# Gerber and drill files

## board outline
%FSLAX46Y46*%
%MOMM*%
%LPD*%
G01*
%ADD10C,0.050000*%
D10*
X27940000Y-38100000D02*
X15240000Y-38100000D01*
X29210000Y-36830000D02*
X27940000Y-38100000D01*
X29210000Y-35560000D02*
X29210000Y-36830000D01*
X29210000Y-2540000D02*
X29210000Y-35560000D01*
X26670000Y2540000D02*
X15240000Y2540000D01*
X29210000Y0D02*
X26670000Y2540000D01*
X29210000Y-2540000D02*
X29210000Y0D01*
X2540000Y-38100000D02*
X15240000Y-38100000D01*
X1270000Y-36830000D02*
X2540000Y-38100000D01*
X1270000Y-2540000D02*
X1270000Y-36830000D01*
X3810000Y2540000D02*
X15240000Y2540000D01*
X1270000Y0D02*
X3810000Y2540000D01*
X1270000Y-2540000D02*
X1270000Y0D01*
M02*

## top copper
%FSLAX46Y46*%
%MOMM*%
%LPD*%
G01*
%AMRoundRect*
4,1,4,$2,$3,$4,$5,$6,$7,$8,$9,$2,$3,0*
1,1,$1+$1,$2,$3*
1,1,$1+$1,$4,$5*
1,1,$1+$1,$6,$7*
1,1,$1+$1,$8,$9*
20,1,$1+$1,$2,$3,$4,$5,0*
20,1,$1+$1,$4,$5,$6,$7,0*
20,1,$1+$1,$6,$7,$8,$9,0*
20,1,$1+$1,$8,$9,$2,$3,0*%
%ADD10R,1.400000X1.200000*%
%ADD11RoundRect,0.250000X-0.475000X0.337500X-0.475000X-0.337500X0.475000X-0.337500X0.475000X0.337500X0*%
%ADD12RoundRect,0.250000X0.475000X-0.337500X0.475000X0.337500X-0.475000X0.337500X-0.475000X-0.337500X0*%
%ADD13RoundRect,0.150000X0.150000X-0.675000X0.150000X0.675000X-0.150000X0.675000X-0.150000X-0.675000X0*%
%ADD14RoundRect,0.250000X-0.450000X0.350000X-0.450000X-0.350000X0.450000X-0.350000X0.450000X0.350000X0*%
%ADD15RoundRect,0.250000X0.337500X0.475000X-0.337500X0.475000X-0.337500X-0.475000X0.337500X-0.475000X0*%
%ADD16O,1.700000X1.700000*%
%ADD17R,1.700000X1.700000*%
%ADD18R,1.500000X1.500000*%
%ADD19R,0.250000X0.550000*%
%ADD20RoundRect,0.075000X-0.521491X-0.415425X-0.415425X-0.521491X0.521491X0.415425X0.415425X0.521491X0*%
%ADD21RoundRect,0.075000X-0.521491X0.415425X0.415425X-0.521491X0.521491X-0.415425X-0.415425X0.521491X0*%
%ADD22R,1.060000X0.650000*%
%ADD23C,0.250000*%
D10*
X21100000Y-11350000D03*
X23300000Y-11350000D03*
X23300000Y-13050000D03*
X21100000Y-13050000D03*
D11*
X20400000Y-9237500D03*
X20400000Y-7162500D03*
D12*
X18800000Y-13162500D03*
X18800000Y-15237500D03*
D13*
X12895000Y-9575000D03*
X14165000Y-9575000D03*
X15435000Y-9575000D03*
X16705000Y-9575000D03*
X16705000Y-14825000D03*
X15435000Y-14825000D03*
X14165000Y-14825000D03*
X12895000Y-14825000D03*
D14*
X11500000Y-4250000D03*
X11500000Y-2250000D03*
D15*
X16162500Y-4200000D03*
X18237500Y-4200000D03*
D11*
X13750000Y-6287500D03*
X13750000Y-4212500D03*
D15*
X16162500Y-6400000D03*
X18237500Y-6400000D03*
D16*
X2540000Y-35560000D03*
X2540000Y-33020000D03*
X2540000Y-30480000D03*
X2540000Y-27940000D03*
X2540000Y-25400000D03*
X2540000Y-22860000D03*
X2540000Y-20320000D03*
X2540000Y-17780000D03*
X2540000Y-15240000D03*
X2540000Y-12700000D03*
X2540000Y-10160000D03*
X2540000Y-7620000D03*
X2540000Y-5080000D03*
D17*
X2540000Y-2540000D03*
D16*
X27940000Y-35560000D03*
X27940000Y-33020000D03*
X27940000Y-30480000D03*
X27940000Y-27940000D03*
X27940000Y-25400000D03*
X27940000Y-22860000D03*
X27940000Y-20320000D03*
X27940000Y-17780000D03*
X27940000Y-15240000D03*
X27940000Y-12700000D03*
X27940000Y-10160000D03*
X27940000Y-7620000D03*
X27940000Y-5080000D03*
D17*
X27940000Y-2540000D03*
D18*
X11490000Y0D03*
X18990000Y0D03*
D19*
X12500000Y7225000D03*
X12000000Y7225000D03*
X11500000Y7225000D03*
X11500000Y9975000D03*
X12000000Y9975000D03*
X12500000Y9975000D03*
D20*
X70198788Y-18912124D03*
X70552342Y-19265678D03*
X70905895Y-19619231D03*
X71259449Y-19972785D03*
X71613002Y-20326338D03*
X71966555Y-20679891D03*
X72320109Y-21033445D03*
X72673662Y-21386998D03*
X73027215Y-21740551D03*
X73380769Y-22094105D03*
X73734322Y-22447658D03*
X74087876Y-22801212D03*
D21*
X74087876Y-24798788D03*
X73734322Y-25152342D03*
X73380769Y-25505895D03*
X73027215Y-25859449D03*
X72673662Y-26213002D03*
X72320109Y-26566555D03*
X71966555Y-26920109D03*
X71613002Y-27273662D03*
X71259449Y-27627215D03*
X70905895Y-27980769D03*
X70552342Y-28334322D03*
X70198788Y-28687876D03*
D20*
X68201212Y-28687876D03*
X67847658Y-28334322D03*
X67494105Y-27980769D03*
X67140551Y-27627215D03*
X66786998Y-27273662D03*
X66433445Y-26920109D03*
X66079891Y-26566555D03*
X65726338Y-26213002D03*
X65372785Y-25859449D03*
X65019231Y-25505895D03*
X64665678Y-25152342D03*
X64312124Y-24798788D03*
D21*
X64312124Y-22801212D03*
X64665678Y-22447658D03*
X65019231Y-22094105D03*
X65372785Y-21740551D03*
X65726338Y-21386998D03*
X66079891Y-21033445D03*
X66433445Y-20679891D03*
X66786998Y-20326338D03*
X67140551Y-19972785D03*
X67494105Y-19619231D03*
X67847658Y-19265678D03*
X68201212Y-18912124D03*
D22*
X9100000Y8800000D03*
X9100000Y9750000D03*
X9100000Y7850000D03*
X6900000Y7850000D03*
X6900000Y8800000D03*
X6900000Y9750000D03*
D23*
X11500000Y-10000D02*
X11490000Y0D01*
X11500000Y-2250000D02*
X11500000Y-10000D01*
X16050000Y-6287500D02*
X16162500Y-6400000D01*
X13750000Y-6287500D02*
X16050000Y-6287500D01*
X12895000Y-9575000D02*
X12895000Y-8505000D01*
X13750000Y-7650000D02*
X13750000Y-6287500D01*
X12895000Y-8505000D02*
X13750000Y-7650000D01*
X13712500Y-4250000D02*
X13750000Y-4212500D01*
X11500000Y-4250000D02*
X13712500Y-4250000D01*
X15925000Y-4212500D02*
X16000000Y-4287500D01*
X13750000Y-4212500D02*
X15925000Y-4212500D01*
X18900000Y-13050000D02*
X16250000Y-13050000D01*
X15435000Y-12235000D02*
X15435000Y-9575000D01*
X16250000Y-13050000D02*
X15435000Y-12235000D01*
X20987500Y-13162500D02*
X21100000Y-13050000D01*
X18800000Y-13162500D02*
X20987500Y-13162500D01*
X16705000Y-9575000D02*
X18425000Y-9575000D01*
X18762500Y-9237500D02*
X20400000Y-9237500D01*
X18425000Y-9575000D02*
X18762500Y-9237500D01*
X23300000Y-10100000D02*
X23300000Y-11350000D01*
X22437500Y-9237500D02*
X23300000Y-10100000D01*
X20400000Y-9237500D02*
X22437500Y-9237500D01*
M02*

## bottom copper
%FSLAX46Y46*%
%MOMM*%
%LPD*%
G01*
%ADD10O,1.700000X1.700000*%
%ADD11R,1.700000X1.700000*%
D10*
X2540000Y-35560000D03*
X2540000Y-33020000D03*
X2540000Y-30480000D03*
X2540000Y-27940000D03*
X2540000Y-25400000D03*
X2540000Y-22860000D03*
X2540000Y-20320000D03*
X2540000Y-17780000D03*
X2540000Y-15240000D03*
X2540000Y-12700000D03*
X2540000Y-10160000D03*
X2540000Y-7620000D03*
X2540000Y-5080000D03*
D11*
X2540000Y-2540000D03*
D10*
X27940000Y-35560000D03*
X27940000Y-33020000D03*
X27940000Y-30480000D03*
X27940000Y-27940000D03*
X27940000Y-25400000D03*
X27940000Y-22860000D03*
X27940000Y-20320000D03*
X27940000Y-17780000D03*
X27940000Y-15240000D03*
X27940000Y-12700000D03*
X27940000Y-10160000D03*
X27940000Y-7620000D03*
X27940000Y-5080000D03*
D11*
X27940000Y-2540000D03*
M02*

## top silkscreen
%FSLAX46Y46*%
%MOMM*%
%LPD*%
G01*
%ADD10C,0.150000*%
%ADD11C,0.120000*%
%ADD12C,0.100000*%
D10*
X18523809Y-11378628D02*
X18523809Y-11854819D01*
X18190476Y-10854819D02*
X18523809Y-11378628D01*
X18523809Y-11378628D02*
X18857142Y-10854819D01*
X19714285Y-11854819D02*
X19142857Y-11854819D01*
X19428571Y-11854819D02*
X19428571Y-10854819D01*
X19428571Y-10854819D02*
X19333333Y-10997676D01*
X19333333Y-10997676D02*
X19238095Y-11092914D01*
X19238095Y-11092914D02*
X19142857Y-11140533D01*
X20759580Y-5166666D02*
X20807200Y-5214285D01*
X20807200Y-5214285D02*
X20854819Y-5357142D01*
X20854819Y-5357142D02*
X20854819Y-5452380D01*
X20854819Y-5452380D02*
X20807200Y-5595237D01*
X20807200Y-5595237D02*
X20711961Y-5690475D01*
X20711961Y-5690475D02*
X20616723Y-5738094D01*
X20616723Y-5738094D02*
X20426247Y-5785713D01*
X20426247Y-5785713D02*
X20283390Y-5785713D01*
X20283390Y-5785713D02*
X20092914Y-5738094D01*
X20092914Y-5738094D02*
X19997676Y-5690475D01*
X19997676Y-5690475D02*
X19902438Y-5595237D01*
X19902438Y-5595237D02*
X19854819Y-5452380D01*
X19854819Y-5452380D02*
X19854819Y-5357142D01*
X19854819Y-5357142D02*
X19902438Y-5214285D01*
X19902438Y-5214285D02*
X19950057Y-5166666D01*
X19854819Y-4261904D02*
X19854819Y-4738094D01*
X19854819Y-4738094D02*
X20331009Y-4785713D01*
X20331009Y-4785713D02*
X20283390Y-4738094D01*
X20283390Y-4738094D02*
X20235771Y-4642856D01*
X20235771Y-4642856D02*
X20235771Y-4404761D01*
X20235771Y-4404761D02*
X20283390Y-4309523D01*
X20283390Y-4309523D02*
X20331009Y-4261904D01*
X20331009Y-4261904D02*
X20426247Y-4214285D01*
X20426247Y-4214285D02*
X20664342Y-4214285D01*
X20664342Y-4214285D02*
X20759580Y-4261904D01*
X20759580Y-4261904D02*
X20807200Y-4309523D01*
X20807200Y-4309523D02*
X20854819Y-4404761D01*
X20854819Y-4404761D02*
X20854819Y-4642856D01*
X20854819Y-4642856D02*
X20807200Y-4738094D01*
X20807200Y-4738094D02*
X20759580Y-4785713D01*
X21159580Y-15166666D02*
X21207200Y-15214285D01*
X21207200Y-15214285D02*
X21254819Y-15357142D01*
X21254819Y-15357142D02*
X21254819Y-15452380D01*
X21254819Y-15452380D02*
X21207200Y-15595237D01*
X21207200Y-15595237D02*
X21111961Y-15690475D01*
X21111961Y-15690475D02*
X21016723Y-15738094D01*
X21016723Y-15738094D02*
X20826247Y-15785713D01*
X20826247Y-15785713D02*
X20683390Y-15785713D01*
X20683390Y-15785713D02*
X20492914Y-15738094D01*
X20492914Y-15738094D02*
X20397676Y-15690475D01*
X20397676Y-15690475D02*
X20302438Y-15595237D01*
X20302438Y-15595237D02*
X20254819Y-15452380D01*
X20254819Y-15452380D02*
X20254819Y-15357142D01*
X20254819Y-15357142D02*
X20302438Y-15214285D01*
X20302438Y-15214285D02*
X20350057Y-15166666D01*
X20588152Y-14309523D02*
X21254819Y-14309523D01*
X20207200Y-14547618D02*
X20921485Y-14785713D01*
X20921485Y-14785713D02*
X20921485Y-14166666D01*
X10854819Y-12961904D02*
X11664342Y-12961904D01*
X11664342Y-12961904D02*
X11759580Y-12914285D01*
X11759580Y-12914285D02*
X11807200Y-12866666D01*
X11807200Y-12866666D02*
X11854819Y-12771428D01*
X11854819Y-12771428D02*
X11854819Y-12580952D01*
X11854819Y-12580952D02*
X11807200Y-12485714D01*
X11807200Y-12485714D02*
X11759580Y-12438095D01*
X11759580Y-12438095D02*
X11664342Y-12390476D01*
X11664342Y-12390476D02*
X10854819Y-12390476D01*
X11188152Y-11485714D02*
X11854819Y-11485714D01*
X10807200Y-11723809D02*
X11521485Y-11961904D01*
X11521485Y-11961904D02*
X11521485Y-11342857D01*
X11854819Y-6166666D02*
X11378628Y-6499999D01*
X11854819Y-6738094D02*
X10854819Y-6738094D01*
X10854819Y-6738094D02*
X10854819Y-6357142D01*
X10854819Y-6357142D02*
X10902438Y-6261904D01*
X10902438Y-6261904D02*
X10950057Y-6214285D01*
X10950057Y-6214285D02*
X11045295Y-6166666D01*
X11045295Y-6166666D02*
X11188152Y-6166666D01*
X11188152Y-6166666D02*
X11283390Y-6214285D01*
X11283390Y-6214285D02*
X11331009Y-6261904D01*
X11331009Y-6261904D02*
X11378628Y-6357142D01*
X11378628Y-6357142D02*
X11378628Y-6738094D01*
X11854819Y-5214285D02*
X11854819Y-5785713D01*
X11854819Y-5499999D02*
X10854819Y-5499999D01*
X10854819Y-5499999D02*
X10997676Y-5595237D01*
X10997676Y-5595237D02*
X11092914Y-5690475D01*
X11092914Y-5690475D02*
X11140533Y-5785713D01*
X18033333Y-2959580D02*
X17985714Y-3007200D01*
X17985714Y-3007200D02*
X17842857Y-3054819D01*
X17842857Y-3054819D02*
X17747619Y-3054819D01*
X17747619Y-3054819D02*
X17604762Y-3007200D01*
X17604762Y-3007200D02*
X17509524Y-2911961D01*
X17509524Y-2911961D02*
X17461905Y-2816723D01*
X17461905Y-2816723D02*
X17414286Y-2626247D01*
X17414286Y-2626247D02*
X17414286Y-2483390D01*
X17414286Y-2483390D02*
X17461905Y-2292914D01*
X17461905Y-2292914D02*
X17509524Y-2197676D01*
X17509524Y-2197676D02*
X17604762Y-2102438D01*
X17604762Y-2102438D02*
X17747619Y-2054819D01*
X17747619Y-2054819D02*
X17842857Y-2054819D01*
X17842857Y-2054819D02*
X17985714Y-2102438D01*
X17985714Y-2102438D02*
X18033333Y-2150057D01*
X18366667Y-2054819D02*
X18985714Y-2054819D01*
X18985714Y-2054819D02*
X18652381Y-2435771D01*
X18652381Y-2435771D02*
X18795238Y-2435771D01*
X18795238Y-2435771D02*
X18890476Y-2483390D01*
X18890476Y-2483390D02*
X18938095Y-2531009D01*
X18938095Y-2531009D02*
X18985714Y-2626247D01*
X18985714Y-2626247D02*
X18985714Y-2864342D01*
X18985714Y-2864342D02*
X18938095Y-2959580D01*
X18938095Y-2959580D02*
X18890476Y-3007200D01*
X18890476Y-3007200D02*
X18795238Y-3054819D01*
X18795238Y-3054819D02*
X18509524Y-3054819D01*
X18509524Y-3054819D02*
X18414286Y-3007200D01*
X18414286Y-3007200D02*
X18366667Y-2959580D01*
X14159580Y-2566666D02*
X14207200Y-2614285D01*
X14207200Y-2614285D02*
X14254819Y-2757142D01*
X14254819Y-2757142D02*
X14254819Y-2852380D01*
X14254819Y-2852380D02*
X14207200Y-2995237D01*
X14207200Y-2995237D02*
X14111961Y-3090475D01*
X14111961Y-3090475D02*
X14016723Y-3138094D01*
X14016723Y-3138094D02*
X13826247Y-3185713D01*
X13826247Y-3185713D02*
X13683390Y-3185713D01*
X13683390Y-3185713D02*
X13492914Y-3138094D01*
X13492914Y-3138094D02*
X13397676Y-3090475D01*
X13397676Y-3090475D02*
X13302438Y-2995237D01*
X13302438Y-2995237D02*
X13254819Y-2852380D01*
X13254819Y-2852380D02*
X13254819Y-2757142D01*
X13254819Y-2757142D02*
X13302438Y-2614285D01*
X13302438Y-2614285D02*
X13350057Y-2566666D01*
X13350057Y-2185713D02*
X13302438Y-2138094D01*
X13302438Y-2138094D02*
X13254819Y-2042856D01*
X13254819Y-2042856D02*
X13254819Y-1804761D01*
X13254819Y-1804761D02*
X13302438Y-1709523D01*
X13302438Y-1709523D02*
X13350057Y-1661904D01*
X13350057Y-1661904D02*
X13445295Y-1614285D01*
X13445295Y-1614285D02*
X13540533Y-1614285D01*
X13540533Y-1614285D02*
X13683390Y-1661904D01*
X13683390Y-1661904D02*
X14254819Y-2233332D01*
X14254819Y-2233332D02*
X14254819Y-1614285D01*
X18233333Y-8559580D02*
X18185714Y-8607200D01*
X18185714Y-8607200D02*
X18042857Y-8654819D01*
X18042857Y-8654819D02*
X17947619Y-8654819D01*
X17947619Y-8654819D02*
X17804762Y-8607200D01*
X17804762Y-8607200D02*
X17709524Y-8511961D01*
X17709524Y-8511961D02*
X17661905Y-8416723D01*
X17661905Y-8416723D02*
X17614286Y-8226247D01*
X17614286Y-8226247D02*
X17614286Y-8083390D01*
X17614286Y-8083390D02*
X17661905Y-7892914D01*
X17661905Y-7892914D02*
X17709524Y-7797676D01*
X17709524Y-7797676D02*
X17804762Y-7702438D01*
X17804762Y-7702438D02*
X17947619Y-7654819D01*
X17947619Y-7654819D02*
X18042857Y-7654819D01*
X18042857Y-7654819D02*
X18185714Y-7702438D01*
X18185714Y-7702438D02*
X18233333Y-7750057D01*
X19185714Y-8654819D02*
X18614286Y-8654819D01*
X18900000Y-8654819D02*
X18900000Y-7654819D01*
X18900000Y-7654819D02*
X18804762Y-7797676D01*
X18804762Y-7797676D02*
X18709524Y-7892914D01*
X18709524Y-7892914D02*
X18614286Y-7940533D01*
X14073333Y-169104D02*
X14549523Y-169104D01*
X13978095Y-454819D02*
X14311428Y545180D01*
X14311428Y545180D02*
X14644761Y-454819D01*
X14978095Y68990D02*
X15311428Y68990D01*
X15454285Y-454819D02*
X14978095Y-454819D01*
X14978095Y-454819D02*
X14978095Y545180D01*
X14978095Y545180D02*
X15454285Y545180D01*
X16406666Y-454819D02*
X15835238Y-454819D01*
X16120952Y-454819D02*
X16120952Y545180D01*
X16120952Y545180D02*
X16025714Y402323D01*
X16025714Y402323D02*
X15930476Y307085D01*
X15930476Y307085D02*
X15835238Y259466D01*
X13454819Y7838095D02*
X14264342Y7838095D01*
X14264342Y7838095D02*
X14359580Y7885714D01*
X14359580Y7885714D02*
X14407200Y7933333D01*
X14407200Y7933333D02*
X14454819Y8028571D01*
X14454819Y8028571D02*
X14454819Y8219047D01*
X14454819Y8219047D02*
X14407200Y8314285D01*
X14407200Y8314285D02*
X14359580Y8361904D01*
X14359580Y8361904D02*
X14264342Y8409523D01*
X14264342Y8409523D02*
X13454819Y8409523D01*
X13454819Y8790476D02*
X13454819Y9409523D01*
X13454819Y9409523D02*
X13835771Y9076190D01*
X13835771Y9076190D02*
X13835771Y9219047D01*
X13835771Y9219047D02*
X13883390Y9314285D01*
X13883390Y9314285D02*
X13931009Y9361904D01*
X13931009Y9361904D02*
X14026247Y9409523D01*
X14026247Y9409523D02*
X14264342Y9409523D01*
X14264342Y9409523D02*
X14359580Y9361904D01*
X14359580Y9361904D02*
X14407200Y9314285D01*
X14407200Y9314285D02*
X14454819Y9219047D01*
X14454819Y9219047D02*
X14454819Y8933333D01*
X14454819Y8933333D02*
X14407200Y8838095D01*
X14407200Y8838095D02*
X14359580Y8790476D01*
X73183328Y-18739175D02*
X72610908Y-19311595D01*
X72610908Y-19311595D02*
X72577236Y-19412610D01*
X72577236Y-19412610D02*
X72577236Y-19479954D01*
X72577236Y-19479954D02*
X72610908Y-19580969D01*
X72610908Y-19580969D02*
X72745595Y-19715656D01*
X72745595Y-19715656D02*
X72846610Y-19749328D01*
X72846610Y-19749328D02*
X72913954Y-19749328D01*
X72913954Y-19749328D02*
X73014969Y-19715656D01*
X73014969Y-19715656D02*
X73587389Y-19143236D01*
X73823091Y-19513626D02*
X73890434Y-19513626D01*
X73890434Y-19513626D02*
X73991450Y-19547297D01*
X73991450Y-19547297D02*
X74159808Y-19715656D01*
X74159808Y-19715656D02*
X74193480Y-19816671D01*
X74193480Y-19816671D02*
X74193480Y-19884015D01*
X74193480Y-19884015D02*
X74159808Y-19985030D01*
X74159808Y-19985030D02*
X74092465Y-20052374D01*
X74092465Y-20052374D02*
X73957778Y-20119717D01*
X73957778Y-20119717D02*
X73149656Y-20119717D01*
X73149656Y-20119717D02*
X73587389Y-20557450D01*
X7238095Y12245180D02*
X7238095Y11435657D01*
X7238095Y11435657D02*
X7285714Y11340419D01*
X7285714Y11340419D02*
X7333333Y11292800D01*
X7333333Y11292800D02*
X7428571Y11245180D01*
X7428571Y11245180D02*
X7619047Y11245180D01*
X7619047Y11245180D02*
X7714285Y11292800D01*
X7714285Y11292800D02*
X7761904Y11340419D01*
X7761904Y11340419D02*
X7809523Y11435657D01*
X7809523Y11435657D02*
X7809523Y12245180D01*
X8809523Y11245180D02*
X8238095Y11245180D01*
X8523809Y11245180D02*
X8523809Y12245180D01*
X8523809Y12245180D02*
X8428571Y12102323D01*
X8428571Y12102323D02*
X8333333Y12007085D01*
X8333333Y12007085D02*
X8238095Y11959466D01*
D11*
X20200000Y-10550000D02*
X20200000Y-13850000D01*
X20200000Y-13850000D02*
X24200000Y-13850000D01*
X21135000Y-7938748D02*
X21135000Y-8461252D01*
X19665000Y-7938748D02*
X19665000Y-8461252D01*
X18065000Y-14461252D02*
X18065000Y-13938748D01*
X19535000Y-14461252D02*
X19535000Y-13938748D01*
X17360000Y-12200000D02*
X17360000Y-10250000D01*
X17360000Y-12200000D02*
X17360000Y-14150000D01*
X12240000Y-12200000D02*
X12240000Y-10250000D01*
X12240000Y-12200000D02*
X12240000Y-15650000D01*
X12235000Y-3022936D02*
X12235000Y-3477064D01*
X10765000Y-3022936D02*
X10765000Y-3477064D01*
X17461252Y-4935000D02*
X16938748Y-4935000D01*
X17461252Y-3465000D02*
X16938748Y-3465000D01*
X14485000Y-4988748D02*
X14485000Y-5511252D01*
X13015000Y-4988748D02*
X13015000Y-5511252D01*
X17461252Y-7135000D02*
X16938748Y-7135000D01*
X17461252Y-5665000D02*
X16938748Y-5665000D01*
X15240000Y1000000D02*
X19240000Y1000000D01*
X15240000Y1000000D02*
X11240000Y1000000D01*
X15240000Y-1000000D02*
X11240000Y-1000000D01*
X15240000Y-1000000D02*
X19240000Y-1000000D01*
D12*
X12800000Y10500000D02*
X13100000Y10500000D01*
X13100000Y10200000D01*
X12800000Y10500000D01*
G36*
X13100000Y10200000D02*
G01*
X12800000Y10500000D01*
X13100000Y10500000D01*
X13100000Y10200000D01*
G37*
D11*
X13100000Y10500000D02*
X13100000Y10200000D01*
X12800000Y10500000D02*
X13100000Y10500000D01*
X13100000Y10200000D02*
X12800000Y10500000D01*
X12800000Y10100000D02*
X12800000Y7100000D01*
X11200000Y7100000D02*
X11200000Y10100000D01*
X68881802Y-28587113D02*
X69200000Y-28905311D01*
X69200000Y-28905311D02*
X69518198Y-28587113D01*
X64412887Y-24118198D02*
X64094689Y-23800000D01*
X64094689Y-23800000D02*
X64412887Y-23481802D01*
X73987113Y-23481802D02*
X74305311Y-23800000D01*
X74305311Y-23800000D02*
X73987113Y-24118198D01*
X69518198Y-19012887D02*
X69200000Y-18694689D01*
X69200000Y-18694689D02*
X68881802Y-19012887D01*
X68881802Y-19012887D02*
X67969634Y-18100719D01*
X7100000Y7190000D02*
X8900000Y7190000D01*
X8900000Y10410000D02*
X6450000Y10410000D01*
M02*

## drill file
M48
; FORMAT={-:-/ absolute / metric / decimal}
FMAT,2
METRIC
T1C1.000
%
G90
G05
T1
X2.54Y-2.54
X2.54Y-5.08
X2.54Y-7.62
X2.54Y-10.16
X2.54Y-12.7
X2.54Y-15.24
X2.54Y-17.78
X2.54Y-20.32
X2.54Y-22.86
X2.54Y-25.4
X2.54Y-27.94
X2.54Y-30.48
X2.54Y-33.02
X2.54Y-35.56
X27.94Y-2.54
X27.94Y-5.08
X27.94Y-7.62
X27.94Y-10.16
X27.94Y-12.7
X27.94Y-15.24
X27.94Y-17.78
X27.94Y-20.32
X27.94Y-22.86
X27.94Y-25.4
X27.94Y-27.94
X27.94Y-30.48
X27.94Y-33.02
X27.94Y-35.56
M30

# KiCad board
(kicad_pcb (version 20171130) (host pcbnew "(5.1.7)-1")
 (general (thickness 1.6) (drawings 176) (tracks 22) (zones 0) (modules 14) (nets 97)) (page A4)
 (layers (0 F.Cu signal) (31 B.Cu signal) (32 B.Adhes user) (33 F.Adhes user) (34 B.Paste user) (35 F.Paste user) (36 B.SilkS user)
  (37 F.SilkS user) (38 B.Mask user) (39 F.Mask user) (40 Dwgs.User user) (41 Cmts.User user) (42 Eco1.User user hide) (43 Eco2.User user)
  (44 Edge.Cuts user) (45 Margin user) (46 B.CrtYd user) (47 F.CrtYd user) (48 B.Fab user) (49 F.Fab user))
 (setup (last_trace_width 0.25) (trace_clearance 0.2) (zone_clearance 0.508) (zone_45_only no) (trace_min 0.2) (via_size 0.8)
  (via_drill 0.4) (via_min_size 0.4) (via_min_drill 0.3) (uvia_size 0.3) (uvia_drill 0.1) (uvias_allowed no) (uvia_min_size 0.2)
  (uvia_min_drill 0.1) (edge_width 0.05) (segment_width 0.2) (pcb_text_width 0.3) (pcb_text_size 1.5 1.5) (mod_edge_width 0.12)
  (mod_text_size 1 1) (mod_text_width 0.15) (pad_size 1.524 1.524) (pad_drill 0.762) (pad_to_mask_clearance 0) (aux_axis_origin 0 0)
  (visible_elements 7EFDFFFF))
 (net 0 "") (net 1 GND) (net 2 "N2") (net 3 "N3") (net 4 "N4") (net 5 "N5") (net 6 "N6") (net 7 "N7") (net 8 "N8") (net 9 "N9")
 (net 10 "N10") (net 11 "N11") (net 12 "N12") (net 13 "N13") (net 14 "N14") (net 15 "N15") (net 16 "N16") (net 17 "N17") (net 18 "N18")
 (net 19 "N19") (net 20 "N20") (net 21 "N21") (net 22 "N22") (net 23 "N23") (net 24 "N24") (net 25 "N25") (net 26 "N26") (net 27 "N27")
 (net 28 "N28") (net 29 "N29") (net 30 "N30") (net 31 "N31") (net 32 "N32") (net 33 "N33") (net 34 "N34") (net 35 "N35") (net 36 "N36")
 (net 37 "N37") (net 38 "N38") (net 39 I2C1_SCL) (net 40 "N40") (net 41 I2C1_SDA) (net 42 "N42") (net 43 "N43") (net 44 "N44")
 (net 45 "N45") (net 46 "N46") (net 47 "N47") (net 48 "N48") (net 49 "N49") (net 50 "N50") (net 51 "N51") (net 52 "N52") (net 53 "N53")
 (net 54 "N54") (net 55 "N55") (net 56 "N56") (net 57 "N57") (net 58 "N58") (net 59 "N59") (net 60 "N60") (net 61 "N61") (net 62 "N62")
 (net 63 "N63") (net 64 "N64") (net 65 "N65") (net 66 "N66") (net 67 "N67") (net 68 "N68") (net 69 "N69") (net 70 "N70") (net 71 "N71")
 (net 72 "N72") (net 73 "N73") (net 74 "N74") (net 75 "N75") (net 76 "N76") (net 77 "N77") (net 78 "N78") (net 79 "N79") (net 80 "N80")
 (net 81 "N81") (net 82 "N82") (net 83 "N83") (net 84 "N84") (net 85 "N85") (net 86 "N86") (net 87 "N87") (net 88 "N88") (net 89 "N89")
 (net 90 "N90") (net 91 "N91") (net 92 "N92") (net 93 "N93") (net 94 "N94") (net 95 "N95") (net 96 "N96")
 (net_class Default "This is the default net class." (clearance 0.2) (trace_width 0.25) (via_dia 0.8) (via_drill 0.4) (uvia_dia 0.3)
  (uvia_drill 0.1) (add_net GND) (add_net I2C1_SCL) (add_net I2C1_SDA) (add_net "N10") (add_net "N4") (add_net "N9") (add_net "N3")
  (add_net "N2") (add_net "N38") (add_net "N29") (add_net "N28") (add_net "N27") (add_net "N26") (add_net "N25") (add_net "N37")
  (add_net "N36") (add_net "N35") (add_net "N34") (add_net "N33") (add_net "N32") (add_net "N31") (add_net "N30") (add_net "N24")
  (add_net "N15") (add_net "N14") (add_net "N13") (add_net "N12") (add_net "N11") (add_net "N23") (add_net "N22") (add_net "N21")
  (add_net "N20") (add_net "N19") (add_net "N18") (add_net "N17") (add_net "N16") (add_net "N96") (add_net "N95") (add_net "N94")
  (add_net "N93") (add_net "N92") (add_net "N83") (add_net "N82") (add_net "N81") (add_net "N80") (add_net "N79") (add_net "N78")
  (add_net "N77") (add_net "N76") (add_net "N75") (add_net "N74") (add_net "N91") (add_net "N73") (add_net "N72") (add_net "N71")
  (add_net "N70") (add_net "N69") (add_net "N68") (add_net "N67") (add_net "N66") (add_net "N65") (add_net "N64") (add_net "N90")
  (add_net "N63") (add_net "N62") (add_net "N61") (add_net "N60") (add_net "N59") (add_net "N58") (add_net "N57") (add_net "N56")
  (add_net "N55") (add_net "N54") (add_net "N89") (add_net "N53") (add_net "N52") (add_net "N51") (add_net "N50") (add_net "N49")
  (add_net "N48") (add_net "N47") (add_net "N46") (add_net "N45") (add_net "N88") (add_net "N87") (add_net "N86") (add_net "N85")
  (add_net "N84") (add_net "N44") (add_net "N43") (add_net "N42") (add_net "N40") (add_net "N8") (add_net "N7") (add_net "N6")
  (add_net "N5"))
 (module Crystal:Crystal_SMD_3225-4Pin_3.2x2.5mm (layer F.Cu) (at 22.2 12.2)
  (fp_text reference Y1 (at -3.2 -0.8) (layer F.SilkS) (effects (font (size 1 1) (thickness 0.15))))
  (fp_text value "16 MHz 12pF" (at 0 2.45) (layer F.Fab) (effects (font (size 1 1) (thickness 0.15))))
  (fp_line (start -2 -1.65) (end -2 1.65) (layer F.SilkS) (width 0.12))
  (fp_line (start -2 1.65) (end 2 1.65) (layer F.SilkS) (width 0.12))
  (pad 4 smd rect (at -1.1 -0.85) (size 1.4 1.2) (layers F.Cu F.Paste F.Mask) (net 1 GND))
  (pad 3 smd rect (at 1.1 -0.85) (size 1.4 1.2) (layers F.Cu F.Paste F.Mask) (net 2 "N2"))
  (pad 2 smd rect (at 1.1 0.85) (size 1.4 1.2) (layers F.Cu F.Paste F.Mask) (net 1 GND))
  (pad 1 smd rect (at -1.1 0.85) (size 1.4 1.2) (layers F.Cu F.Paste F.Mask) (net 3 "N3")))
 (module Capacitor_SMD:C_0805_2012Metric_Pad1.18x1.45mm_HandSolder (layer F.Cu) (at 20.4 8.2 270)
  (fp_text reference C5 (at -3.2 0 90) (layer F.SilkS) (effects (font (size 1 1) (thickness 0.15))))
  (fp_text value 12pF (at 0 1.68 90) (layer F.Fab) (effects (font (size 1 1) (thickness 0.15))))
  (fp_line (start -0.261252 -0.735) (end 0.261252 -0.735) (layer F.SilkS) (width 0.12))
  (fp_line (start -0.261252 0.735) (end 0.261252 0.735) (layer F.SilkS) (width 0.12))
  (pad 2 smd roundrect (at 1.0375 0 270) (size 1.175 1.45) (layers F.Cu F.Paste F.Mask) (roundrect_rratio 0.212766) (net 2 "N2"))
  (pad 1 smd roundrect (at -1.0375 0 270) (size 1.175 1.45) (layers F.Cu F.Paste F.Mask) (roundrect_rratio 0.212766) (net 1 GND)))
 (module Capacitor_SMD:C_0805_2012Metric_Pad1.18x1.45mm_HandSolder (layer F.Cu) (at 18.8 14.2 90)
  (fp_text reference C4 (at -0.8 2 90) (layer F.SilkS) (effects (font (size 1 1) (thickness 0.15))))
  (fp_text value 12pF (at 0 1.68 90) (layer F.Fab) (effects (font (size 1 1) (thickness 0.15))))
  (fp_line (start -0.261252 -0.735) (end 0.261252 -0.735) (layer F.SilkS) (width 0.12))
  (fp_line (start -0.261252 0.735) (end 0.261252 0.735) (layer F.SilkS) (width 0.12))
  (pad 2 smd roundrect (at 1.0375 0 90) (size 1.175 1.45) (layers F.Cu F.Paste F.Mask) (roundrect_rratio 0.212766) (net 3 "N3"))
  (pad 1 smd roundrect (at -1.0375 0 90) (size 1.175 1.45) (layers F.Cu F.Paste F.Mask) (roundrect_rratio 0.212766) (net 1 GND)))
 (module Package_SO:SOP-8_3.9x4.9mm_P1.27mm (layer F.Cu) (at 14.8 12.2 90)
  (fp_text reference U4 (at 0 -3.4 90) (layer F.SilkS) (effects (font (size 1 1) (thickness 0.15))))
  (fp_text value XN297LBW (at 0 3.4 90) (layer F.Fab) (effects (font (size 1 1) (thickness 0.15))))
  (fp_line (start 0 2.56) (end 1.95 2.56) (layer F.SilkS) (width 0.12))
  (fp_line (start 0 2.56) (end -1.95 2.56) (layer F.SilkS) (width 0.12))
  (fp_line (start 0 -2.56) (end 1.95 -2.56) (layer F.SilkS) (width 0.12))
  (fp_line (start 0 -2.56) (end -3.45 -2.56) (layer F.SilkS) (width 0.12))
  (pad 8 smd roundrect (at 2.625 -1.905 90) (size 1.65 0.6) (layers F.Cu F.Paste F.Mask) (roundrect_rratio 0.25) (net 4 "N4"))
  (pad 7 smd roundrect (at 2.625 -0.635 90) (size 1.65 0.6) (layers F.Cu F.Paste F.Mask) (roundrect_rratio 0.25) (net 1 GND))
  (pad 6 smd roundrect (at 2.625 0.635 90) (size 1.65 0.6) (layers F.Cu F.Paste F.Mask) (roundrect_rratio 0.25) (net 3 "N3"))
  (pad 5 smd roundrect (at 2.625 1.905 90) (size 1.65 0.6) (layers F.Cu F.Paste F.Mask) (roundrect_rratio 0.25) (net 2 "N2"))
  (pad 4 smd roundrect (at -2.625 1.905 90) (size 1.65 0.6) (layers F.Cu F.Paste F.Mask) (roundrect_rratio 0.25) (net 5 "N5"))
  (pad 3 smd roundrect (at -2.625 0.635 90) (size 1.65 0.6) (layers F.Cu F.Paste F.Mask) (roundrect_rratio 0.25) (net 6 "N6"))
  (pad 2 smd roundrect (at -2.625 -0.635 90) (size 1.65 0.6) (layers F.Cu F.Paste F.Mask) (roundrect_rratio 0.25) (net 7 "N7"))
  (pad 1 smd roundrect (at -2.625 -1.905 90) (size 1.65 0.6) (layers F.Cu F.Paste F.Mask) (roundrect_rratio 0.25) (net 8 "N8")))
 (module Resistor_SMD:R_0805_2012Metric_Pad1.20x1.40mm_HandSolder (layer F.Cu) (at 11.5 3.25 270)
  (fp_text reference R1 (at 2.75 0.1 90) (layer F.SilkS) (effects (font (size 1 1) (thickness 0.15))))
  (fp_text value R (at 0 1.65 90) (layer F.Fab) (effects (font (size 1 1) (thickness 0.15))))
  (fp_line (start -0.227064 -0.735) (end 0.227064 -0.735) (layer F.SilkS) (width 0.12))
  (fp_line (start -0.227064 0.735) (end 0.227064 0.735) (layer F.SilkS) (width 0.12))
  (pad 2 smd roundrect (at 1 0 270) (size 1.2 1.4) (layers F.Cu F.Paste F.Mask) (roundrect_rratio 0.208333) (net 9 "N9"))
  (pad 1 smd roundrect (at -1 0 270) (size 1.2 1.4) (layers F.Cu F.Paste F.Mask) (roundrect_rratio 0.208333) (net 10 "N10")))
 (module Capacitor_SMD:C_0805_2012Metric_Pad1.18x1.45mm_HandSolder (layer F.Cu) (at 17.2 4.2 180)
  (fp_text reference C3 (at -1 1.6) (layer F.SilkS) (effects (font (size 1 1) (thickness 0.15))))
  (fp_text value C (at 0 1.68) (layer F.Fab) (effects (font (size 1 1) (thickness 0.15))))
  (fp_line (start -0.261252 -0.735) (end 0.261252 -0.735) (layer F.SilkS) (width 0.12))
  (fp_line (start -0.261252 0.735) (end 0.261252 0.735) (layer F.SilkS) (width 0.12))
  (pad 2 smd roundrect (at 1.0375 0 180) (size 1.175 1.45) (layers F.Cu F.Paste F.Mask) (roundrect_rratio 0.212766) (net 9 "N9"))
  (pad 1 smd roundrect (at -1.0375 0 180) (size 1.175 1.45) (layers F.Cu F.Paste F.Mask) (roundrect_rratio 0.212766) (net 1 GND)))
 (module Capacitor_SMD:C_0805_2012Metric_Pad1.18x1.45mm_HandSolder (layer F.Cu) (at 13.75 5.25 270)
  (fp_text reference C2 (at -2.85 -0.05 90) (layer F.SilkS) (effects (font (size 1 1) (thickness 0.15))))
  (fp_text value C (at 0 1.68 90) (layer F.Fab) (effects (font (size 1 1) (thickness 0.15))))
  (fp_line (start -0.261252 -0.735) (end 0.261252 -0.735) (layer F.SilkS) (width 0.12))
  (fp_line (start -0.261252 0.735) (end 0.261252 0.735) (layer F.SilkS) (width 0.12))
  (pad 2 smd roundrect (at 1.0375 0 270) (size 1.175 1.45) (layers F.Cu F.Paste F.Mask) (roundrect_rratio 0.212766) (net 4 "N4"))
  (pad 1 smd roundrect (at -1.0375 0 270) (size 1.175 1.45) (layers F.Cu F.Paste F.Mask) (roundrect_rratio 0.212766) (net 9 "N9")))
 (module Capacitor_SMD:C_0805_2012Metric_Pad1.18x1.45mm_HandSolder (layer F.Cu) (at 17.2 6.4 180)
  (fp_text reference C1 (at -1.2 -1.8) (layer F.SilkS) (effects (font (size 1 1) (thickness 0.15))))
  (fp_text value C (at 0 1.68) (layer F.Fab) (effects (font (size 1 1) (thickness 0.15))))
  (fp_line (start -0.261252 -0.735) (end 0.261252 -0.735) (layer F.SilkS) (width 0.12))
  (fp_line (start -0.261252 0.735) (end 0.261252 0.735) (layer F.SilkS) (width 0.12))
  (pad 2 smd roundrect (at 1.0375 0 180) (size 1.175 1.45) (layers F.Cu F.Paste F.Mask) (roundrect_rratio 0.212766) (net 4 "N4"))
  (pad 1 smd roundrect (at -1.0375 0 180) (size 1.175 1.45) (layers F.Cu F.Paste F.Mask) (roundrect_rratio 0.212766) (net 1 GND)))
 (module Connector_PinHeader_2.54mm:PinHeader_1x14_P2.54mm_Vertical (layer B.Cu) (at 2.54 2.54 180)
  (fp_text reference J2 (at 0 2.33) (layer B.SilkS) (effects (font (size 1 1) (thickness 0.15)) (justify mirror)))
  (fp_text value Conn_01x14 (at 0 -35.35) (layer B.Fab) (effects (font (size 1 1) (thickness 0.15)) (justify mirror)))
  (pad 14 thru_hole oval (at 0 -33.02 180) (size 1.7 1.7) (drill 1) (layers *.Cu *.Mask) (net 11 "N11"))
  (pad 13 thru_hole oval (at 0 -30.48 180) (size 1.7 1.7) (drill 1) (layers *.Cu *.Mask) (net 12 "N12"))
  (pad 12 thru_hole oval (at 0 -27.94 180) (size 1.7 1.7) (drill 1) (layers *.Cu *.Mask) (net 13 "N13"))
  (pad 11 thru_hole oval (at 0 -25.4 180) (size 1.7 1.7) (drill 1) (layers *.Cu *.Mask) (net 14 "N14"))
  (pad 10 thru_hole oval (at 0 -22.86 180) (size 1.7 1.7) (drill 1) (layers *.Cu *.Mask) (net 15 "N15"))
  (pad 9 thru_hole oval (at 0 -20.32 180) (size 1.7 1.7) (drill 1) (layers *.Cu *.Mask) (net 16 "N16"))
  (pad 8 thru_hole oval (at 0 -17.78 180) (size 1.7 1.7) (drill 1) (layers *.Cu *.Mask) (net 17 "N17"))
  (pad 7 thru_hole oval (at 0 -15.24 180) (size 1.7 1.7) (drill 1) (layers *.Cu *.Mask) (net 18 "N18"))
  (pad 6 thru_hole oval (at 0 -12.7 180) (size 1.7 1.7) (drill 1) (layers *.Cu *.Mask) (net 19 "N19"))
  (pad 5 thru_hole oval (at 0 -10.16 180) (size 1.7 1.7) (drill 1) (layers *.Cu *.Mask) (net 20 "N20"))
  (pad 4 thru_hole oval (at 0 -7.62 180) (size 1.7 1.7) (drill 1) (layers *.Cu *.Mask) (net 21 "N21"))
  (pad 3 thru_hole oval (at 0 -5.08 180) (size 1.7 1.7) (drill 1) (layers *.Cu *.Mask) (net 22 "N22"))
  (pad 2 thru_hole oval (at 0 -2.54 180) (size 1.7 1.7) (drill 1) (layers *.Cu *.Mask) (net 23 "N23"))
  (pad 1 thru_hole rect (at 0 0 180) (size 1.7 1.7) (drill 1) (layers *.Cu *.Mask) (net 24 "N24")))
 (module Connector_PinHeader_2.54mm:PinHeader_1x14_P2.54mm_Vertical (layer B.Cu) (at 27.94 2.54 180)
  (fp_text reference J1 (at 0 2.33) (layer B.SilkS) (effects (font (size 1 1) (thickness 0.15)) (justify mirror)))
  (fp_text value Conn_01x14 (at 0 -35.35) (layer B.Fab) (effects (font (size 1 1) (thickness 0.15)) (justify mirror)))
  (pad 14 thru_hole oval (at 0 -33.02 180) (size 1.7 1.7) (drill 1) (layers *.Cu *.Mask) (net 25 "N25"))
  (pad 13 thru_hole oval (at 0 -30.48 180) (size 1.7 1.7) (drill 1) (layers *.Cu *.Mask) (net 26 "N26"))
  (pad 12 thru_hole oval (at 0 -27.94 180) (size 1.7 1.7) (drill 1) (layers *.Cu *.Mask) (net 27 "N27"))
  (pad 11 thru_hole oval (at 0 -25.4 180) (size 1.7 1.7) (drill 1) (layers *.Cu *.Mask) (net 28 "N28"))
  (pad 10 thru_hole oval (at 0 -22.86 180) (size 1.7 1.7) (drill 1) (layers *.Cu *.Mask) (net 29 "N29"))
  (pad 9 thru_hole oval (at 0 -20.32 180) (size 1.7 1.7) (drill 1) (layers *.Cu *.Mask) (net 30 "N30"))
  (pad 8 thru_hole oval (at 0 -17.78 180) (size 1.7 1.7) (drill 1) (layers *.Cu *.Mask) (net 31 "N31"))
  (pad 7 thru_hole oval (at 0 -15.24 180) (size 1.7 1.7) (drill 1) (layers *.Cu *.Mask) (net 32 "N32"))
  (pad 6 thru_hole oval (at 0 -12.7 180) (size 1.7 1.7) (drill 1) (layers *.Cu *.Mask) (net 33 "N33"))
  (pad 5 thru_hole oval (at 0 -10.16 180) (size 1.7 1.7) (drill 1) (layers *.Cu *.Mask) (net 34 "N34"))
  (pad 4 thru_hole oval (at 0 -7.62 180) (size 1.7 1.7) (drill 1) (layers *.Cu *.Mask) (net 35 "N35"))
  (pad 3 thru_hole oval (at 0 -5.08 180) (size 1.7 1.7) (drill 1) (layers *.Cu *.Mask) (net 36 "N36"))
  (pad 2 thru_hole oval (at 0 -2.54 180) (size 1.7 1.7) (drill 1) (layers *.Cu *.Mask) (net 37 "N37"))
  (pad 1 thru_hole rect (at 0 0 180) (size 1.7 1.7) (drill 1) (layers *.Cu *.Mask) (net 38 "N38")))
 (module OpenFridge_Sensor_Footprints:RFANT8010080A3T (layer F.Cu) (at 15.24 0 180)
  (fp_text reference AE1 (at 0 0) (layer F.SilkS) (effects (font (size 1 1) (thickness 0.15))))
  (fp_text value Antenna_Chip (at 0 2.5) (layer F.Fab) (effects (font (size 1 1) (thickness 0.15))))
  (fp_line (start 0 1) (end -4 1) (layer F.SilkS) (width 0.12)) (fp_line (start 0 1) (end 4 1) (layer F.SilkS) (width 0.12))
  (fp_line (start 0 -1) (end 4 -1) (layer F.SilkS) (width 0.12))
  (fp_line (start 0 -1) (end -4 -1) (layer F.SilkS) (width 0.12))
  (pad 2 smd rect (at 3.75 0 180) (size 1.5 1.5) (layers F.Cu F.Paste F.Mask) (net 10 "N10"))
  (pad 1 smd rect (at -3.75 0 180) (size 1.5 1.5) (layers F.Cu F.Paste F.Mask) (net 1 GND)))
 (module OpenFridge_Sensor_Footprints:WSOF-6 (layer F.Cu) (at 12 -8.6 270)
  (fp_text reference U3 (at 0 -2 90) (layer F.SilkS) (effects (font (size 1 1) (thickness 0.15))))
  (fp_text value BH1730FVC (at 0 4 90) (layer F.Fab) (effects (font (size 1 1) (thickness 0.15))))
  (fp_poly (pts (xy -1.9 -0.8) (xy -1.9 -1.1) (xy -1.6 -1.1)) (layer F.SilkS) (width 0.1))
  (fp_line (start -1.9 -1.1) (end -1.6 -1.1) (layer F.SilkS) (width 0.12))
  (fp_line (start -1.9 -0.8) (end -1.9 -1.1) (layer F.SilkS) (width 0.12))
  (fp_line (start -1.6 -1.1) (end -1.9 -0.8) (layer F.SilkS) (width 0.12))
  (fp_line (start -1.5 -0.8) (end 1.5 -0.8) (layer F.SilkS) (width 0.12))
  (fp_line (start 1.5 0.8) (end -1.5 0.8) (layer F.SilkS) (width 0.12))
  (pad 6 smd rect (at 1.375 -0.5 270) (size 0.55 0.25) (layers F.Cu F.Paste F.Mask) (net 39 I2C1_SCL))
  (pad 5 smd rect (at 1.375 0 270) (size 0.55 0.25) (layers F.Cu F.Paste F.Mask) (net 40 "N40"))
  (pad 4 smd rect (at 1.375 0.5 270) (size 0.55 0.25) (layers F.Cu F.Paste F.Mask) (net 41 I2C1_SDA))
  (pad 3 smd rect (at -1.375 0.5 270) (size 0.55 0.25) (layers F.Cu F.Paste F.Mask) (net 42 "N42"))
  (pad 2 smd rect (at -1.375 0 270) (size 0.55 0.25) (layers F.Cu F.Paste F.Mask) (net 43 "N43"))
  (pad 1 smd rect (at -1.375 -0.5 270) (size 0.55 0.25) (layers F.Cu F.Paste F.Mask) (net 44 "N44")))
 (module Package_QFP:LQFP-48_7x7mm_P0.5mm (layer F.Cu) (at 69.2 23.8 315)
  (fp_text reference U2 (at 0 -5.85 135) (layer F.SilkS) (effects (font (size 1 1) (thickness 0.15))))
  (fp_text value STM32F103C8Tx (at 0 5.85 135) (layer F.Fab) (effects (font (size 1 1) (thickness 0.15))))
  (fp_line (start 3.16 3.61) (end 3.61 3.61) (layer F.SilkS) (width 0.12))
  (fp_line (start 3.61 3.61) (end 3.61 3.16) (layer F.SilkS) (width 0.12))
  (fp_line (start -3.16 3.61) (end -3.61 3.61) (layer F.SilkS) (width 0.12))
  (fp_line (start -3.61 3.61) (end -3.61 3.16) (layer F.SilkS) (width 0.12))
  (fp_line (start 3.16 -3.61) (end 3.61 -3.61) (layer F.SilkS) (width 0.12))
  (fp_line (start 3.61 -3.61) (end 3.61 -3.16) (layer F.SilkS) (width 0.12))
  (fp_line (start -3.16 -3.61) (end -3.61 -3.61) (layer F.SilkS) (width 0.12))
  (fp_line (start -3.61 -3.61) (end -3.61 -3.16) (layer F.SilkS) (width 0.12))
  (fp_line (start -3.61 -3.16) (end -4.9 -3.16) (layer F.SilkS) (width 0.12))
  (pad 48 smd roundrect (at -2.75 -4.1625 315) (size 0.3 1.475) (layers F.Cu F.Paste F.Mask) (roundrect_rratio 0.25) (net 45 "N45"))
  (pad 47 smd roundrect (at -2.25 -4.1625 315) (size 0.3 1.475) (layers F.Cu F.Paste F.Mask) (roundrect_rratio 0.25) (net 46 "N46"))
  (pad 46 smd roundrect (at -1.75 -4.1625 315) (size 0.3 1.475) (layers F.Cu F.Paste F.Mask) (roundrect_rratio 0.25) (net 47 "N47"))
  (pad 45 smd roundrect (at -1.25 -4.1625 315) (size 0.3 1.475) (layers F.Cu F.Paste F.Mask) (roundrect_rratio 0.25) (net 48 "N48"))
  (pad 44 smd roundrect (at -0.75 -4.1625 315) (size 0.3 1.475) (layers F.Cu F.Paste F.Mask) (roundrect_rratio 0.25) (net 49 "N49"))
  (pad 43 smd roundrect (at -0.25 -4.1625 315) (size 0.3 1.475) (layers F.Cu F.Paste F.Mask) (roundrect_rratio 0.25) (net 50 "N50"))
  (pad 42 smd roundrect (at 0.25 -4.1625 315) (size 0.3 1.475) (layers F.Cu F.Paste F.Mask) (roundrect_rratio 0.25) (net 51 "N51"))
  (pad 41 smd roundrect (at 0.75 -4.1625 315) (size 0.3 1.475) (layers F.Cu F.Paste F.Mask) (roundrect_rratio 0.25) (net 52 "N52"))
  (pad 40 smd roundrect (at 1.25 -4.1625 315) (size 0.3 1.475) (layers F.Cu F.Paste F.Mask) (roundrect_rratio 0.25) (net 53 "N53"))
  (pad 39 smd roundrect (at 1.75 -4.1625 315) (size 0.3 1.475) (layers F.Cu F.Paste F.Mask) (roundrect_rratio 0.25) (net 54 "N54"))
  (pad 38 smd roundrect (at 2.25 -4.1625 315) (size 0.3 1.475) (layers F.Cu F.Paste F.Mask) (roundrect_rratio 0.25) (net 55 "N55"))
  (pad 37 smd roundrect (at 2.75 -4.1625 315) (size 0.3 1.475) (layers F.Cu F.Paste F.Mask) (roundrect_rratio 0.25) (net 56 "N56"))
  (pad 36 smd roundrect (at 4.1625 -2.75 315) (size 1.475 0.3) (layers F.Cu F.Paste F.Mask) (roundrect_rratio 0.25) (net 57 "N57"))
  (pad 35 smd roundrect (at 4.1625 -2.25 315) (size 1.475 0.3) (layers F.Cu F.Paste F.Mask) (roundrect_rratio 0.25) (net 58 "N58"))
  (pad 34 smd roundrect (at 4.1625 -1.75 315) (size 1.475 0.3) (layers F.Cu F.Paste F.Mask) (roundrect_rratio 0.25) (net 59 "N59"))
  (pad 33 smd roundrect (at 4.1625 -1.25 315) (size 1.475 0.3) (layers F.Cu F.Paste F.Mask) (roundrect_rratio 0.25) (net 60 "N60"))
  (pad 32 smd roundrect (at 4.1625 -0.75 315) (size 1.475 0.3) (layers F.Cu F.Paste F.Mask) (roundrect_rratio 0.25) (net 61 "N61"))
  (pad 31 smd roundrect (at 4.1625 -0.25 315) (size 1.475 0.3) (layers F.Cu F.Paste F.Mask) (roundrect_rratio 0.25) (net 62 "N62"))
  (pad 30 smd roundrect (at 4.1625 0.25 315) (size 1.475 0.3) (layers F.Cu F.Paste F.Mask) (roundrect_rratio 0.25) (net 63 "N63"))
  (pad 29 smd roundrect (at 4.1625 0.75 315) (size 1.475 0.3) (layers F.Cu F.Paste F.Mask) (roundrect_rratio 0.25) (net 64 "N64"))
  (pad 28 smd roundrect (at 4.1625 1.25 315) (size 1.475 0.3) (layers F.Cu F.Paste F.Mask) (roundrect_rratio 0.25) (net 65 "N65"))
  (pad 27 smd roundrect (at 4.1625 1.75 315) (size 1.475 0.3) (layers F.Cu F.Paste F.Mask) (roundrect_rratio 0.25) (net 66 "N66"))
  (pad 26 smd roundrect (at 4.1625 2.25 315) (size 1.475 0.3) (layers F.Cu F.Paste F.Mask) (roundrect_rratio 0.25) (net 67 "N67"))
  (pad 25 smd roundrect (at 4.1625 2.75 315) (size 1.475 0.3) (layers F.Cu F.Paste F.Mask) (roundrect_rratio 0.25) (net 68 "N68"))
  (pad 24 smd roundrect (at 2.75 4.1625 315) (size 0.3 1.475) (layers F.Cu F.Paste F.Mask) (roundrect_rratio 0.25) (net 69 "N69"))
  (pad 23 smd roundrect (at 2.25 4.1625 315) (size 0.3 1.475) (layers F.Cu F.Paste F.Mask) (roundrect_rratio 0.25) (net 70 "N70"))
  (pad 22 smd roundrect (at 1.75 4.1625 315) (size 0.3 1.475) (layers F.Cu F.Paste F.Mask) (roundrect_rratio 0.25) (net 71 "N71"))
  (pad 21 smd roundrect (at 1.25 4.1625 315) (size 0.3 1.475) (layers F.Cu F.Paste F.Mask) (roundrect_rratio 0.25) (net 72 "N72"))
  (pad 20 smd roundrect (at 0.75 4.1625 315) (size 0.3 1.475) (layers F.Cu F.Paste F.Mask) (roundrect_rratio 0.25) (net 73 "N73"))
  (pad 19 smd roundrect (at 0.25 4.1625 315) (size 0.3 1.475) (layers F.Cu F.Paste F.Mask) (roundrect_rratio 0.25) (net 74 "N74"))
  (pad 18 smd roundrect (at -0.25 4.1625 315) (size 0.3 1.475) (layers F.Cu F.Paste F.Mask) (roundrect_rratio 0.25) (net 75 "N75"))
  (pad 17 smd roundrect (at -0.75 4.1625 315) (size 0.3 1.475) (layers F.Cu F.Paste F.Mask) (roundrect_rratio 0.25) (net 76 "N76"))
  (pad 16 smd roundrect (at -1.25 4.1625 315) (size 0.3 1.475) (layers F.Cu F.Paste F.Mask) (roundrect_rratio 0.25) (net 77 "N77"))
  (pad 15 smd roundrect (at -1.75 4.1625 315) (size 0.3 1.475) (layers F.Cu F.Paste F.Mask) (roundrect_rratio 0.25) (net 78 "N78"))
  (pad 14 smd roundrect (at -2.25 4.1625 315) (size 0.3 1.475) (layers F.Cu F.Paste F.Mask) (roundrect_rratio 0.25) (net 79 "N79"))
  (pad 13 smd roundrect (at -2.75 4.1625 315) (size 0.3 1.475) (layers F.Cu F.Paste F.Mask) (roundrect_rratio 0.25) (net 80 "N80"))
  (pad 12 smd roundrect (at -4.1625 2.75 315) (size 1.475 0.3) (layers F.Cu F.Paste F.Mask) (roundrect_rratio 0.25) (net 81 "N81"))
  (pad 11 smd roundrect (at -4.1625 2.25 315) (size 1.475 0.3) (layers F.Cu F.Paste F.Mask) (roundrect_rratio 0.25) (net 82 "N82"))
  (pad 10 smd roundrect (at -4.1625 1.75 315) (size 1.475 0.3) (layers F.Cu F.Paste F.Mask) (roundrect_rratio 0.25) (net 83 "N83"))
  (pad 9 smd roundrect (at -4.1625 1.25 315) (size 1.475 0.3) (layers F.Cu F.Paste F.Mask) (roundrect_rratio 0.25) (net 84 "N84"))
  (pad 8 smd roundrect (at -4.1625 0.75 315) (size 1.475 0.3) (layers F.Cu F.Paste F.Mask) (roundrect_rratio 0.25) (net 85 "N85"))
  (pad 7 smd roundrect (at -4.1625 0.25 315) (size 1.475 0.3) (layers F.Cu F.Paste F.Mask) (roundrect_rratio 0.25) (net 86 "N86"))
  (pad 6 smd roundrect (at -4.1625 -0.25 315) (size 1.475 0.3) (layers F.Cu F.Paste F.Mask) (roundrect_rratio 0.25) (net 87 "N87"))
  (pad 5 smd roundrect (at -4.1625 -0.75 315) (size 1.475 0.3) (layers F.Cu F.Paste F.Mask) (roundrect_rratio 0.25) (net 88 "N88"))
  (pad 4 smd roundrect (at -4.1625 -1.25 315) (size 1.475 0.3) (layers F.Cu F.Paste F.Mask) (roundrect_rratio 0.25) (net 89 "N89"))
  (pad 3 smd roundrect (at -4.1625 -1.75 315) (size 1.475 0.3) (layers F.Cu F.Paste F.Mask) (roundrect_rratio 0.25) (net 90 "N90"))
  (pad 2 smd roundrect (at -4.1625 -2.25 315) (size 1.475 0.3) (layers F.Cu F.Paste F.Mask) (roundrect_rratio 0.25) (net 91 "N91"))
  (pad 1 smd roundrect (at -4.1625 -2.75 315) (size 1.475 0.3) (layers F.Cu F.Paste F.Mask) (roundrect_rratio 0.25) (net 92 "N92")))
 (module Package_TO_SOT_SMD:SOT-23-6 (layer F.Cu) (at 8 -8.8)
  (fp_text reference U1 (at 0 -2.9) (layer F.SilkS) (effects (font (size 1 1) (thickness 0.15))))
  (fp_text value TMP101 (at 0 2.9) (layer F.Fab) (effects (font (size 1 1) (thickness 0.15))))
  (fp_line (start -0.9 1.61) (end 0.9 1.61) (layer F.SilkS) (width 0.12))
  (fp_line (start 0.9 -1.61) (end -1.55 -1.61) (layer F.SilkS) (width 0.12))
  (pad 5 smd rect (at 1.1 0) (size 1.06 0.65) (layers F.Cu F.Paste F.Mask) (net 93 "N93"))
  (pad 6 smd rect (at 1.1 -0.95) (size 1.06 0.65) (layers F.Cu F.Paste F.Mask) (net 41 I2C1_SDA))
  (pad 4 smd rect (at 1.1 0.95) (size 1.06 0.65) (layers F.Cu F.Paste F.Mask) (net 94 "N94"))
  (pad 3 smd rect (at -1.1 0.95) (size 1.06 0.65) (layers F.Cu F.Paste F.Mask) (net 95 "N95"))
  (pad 2 smd rect (at -1.1 0) (size 1.06 0.65) (layers F.Cu F.Paste F.Mask) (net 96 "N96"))
  (pad 1 smd rect (at -1.1 -0.95) (size 1.06 0.65) (layers F.Cu F.Paste F.Mask) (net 39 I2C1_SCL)))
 (gr_line (start 27.94 38.1) (end 15.24 38.1) (layer Edge.Cuts) (width 0.05))
 (gr_line (start 29.21 36.83) (end 27.94 38.1) (layer Edge.Cuts) (width 0.05))
 (gr_line (start 29.21 35.56) (end 29.21 36.83) (layer Edge.Cuts) (width 0.05))
 (gr_line (start 29.21 2.54) (end 29.21 35.56) (layer Edge.Cuts) (width 0.05))
 (gr_line (start 26.67 -2.54) (end 15.24 -2.54) (layer Edge.Cuts) (width 0.05))
 (gr_line (start 29.21 0) (end 26.67 -2.54) (layer Edge.Cuts) (width 0.05))
 (gr_line (start 29.21 2.54) (end 29.21 0) (layer Edge.Cuts) (width 0.05))
 (gr_line (start 2.54 38.1) (end 15.24 38.1) (layer Edge.Cuts) (width 0.05))
 (gr_line (start 1.27 36.83) (end 2.54 38.1) (layer Edge.Cuts) (width 0.05))
 (gr_line (start 1.27 2.54) (end 1.27 36.83) (layer Edge.Cuts) (width 0.05))
 (gr_line (start 3.81 -2.54) (end 15.24 -2.54) (layer Edge.Cuts) (width 0.05))
 (gr_line (start 1.27 0) (end 3.81 -2.54) (layer Edge.Cuts) (width 0.05))
 (gr_line (start 1.27 2.54) (end 1.27 0) (layer Edge.Cuts) (width 0.05))
 (segment (start 11.5 0.01) (end 11.49 0) (width 0.25) (layer F.Cu) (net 10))
 (segment (start 11.5 2.25) (end 11.5 0.01) (width 0.25) (layer F.Cu) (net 10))
 (segment (start 16.05 6.2875) (end 16.1625 6.4) (width 0.25) (layer F.Cu) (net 4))
 (segment (start 13.75 6.2875) (end 16.05 6.2875) (width 0.25) (layer F.Cu) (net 4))
 (segment (start 12.895 9.575) (end 12.895 8.505) (width 0.25) (layer F.Cu) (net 4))
 (segment (start 13.75 7.65) (end 13.75 6.2875) (width 0.25) (layer F.Cu) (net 4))
 (segment (start 12.895 8.505) (end 13.75 7.65) (width 0.25) (layer F.Cu) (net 4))
 (segment (start 13.7125 4.25) (end 13.75 4.2125) (width 0.25) (layer F.Cu) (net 9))
 (segment (start 11.5 4.25) (end 13.7125 4.25) (width 0.25) (layer F.Cu) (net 9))
 (segment (start 15.925 4.2125) (end 16 4.2875) (width 0.25) (layer F.Cu) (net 9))
 (segment (start 13.75 4.2125) (end 15.925 4.2125) (width 0.25) (layer F.Cu) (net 9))
 (segment (start 18.9 13.05) (end 16.25 13.05) (width 0.25) (layer F.Cu) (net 3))
 (segment (start 15.435 12.235) (end 15.435 9.575) (width 0.25) (layer F.Cu) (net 3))
 (segment (start 16.25 13.05) (end 15.435 12.235) (width 0.25) (layer F.Cu) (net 3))
 (segment (start 20.9875 13.1625) (end 21.1 13.05) (width 0.25) (layer F.Cu) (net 3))
 (segment (start 18.8 13.1625) (end 20.9875 13.1625) (width 0.25) (layer F.Cu) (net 3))
 (segment (start 16.705 9.575) (end 18.425 9.575) (width 0.25) (layer F.Cu) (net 2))
 (segment (start 18.7625 9.2375) (end 20.4 9.2375) (width 0.25) (layer F.Cu) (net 2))
 (segment (start 18.425 9.575) (end 18.7625 9.2375) (width 0.25) (layer F.Cu) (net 2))
 (segment (start 23.3 10.1) (end 23.3 11.35) (width 0.25) (layer F.Cu) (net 2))
 (segment (start 22.4375 9.2375) (end 23.3 10.1) (width 0.25) (layer F.Cu) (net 2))
 (segment (start 20.4 9.2375) (end 22.4375 9.2375) (width 0.25) (layer F.Cu) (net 2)))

